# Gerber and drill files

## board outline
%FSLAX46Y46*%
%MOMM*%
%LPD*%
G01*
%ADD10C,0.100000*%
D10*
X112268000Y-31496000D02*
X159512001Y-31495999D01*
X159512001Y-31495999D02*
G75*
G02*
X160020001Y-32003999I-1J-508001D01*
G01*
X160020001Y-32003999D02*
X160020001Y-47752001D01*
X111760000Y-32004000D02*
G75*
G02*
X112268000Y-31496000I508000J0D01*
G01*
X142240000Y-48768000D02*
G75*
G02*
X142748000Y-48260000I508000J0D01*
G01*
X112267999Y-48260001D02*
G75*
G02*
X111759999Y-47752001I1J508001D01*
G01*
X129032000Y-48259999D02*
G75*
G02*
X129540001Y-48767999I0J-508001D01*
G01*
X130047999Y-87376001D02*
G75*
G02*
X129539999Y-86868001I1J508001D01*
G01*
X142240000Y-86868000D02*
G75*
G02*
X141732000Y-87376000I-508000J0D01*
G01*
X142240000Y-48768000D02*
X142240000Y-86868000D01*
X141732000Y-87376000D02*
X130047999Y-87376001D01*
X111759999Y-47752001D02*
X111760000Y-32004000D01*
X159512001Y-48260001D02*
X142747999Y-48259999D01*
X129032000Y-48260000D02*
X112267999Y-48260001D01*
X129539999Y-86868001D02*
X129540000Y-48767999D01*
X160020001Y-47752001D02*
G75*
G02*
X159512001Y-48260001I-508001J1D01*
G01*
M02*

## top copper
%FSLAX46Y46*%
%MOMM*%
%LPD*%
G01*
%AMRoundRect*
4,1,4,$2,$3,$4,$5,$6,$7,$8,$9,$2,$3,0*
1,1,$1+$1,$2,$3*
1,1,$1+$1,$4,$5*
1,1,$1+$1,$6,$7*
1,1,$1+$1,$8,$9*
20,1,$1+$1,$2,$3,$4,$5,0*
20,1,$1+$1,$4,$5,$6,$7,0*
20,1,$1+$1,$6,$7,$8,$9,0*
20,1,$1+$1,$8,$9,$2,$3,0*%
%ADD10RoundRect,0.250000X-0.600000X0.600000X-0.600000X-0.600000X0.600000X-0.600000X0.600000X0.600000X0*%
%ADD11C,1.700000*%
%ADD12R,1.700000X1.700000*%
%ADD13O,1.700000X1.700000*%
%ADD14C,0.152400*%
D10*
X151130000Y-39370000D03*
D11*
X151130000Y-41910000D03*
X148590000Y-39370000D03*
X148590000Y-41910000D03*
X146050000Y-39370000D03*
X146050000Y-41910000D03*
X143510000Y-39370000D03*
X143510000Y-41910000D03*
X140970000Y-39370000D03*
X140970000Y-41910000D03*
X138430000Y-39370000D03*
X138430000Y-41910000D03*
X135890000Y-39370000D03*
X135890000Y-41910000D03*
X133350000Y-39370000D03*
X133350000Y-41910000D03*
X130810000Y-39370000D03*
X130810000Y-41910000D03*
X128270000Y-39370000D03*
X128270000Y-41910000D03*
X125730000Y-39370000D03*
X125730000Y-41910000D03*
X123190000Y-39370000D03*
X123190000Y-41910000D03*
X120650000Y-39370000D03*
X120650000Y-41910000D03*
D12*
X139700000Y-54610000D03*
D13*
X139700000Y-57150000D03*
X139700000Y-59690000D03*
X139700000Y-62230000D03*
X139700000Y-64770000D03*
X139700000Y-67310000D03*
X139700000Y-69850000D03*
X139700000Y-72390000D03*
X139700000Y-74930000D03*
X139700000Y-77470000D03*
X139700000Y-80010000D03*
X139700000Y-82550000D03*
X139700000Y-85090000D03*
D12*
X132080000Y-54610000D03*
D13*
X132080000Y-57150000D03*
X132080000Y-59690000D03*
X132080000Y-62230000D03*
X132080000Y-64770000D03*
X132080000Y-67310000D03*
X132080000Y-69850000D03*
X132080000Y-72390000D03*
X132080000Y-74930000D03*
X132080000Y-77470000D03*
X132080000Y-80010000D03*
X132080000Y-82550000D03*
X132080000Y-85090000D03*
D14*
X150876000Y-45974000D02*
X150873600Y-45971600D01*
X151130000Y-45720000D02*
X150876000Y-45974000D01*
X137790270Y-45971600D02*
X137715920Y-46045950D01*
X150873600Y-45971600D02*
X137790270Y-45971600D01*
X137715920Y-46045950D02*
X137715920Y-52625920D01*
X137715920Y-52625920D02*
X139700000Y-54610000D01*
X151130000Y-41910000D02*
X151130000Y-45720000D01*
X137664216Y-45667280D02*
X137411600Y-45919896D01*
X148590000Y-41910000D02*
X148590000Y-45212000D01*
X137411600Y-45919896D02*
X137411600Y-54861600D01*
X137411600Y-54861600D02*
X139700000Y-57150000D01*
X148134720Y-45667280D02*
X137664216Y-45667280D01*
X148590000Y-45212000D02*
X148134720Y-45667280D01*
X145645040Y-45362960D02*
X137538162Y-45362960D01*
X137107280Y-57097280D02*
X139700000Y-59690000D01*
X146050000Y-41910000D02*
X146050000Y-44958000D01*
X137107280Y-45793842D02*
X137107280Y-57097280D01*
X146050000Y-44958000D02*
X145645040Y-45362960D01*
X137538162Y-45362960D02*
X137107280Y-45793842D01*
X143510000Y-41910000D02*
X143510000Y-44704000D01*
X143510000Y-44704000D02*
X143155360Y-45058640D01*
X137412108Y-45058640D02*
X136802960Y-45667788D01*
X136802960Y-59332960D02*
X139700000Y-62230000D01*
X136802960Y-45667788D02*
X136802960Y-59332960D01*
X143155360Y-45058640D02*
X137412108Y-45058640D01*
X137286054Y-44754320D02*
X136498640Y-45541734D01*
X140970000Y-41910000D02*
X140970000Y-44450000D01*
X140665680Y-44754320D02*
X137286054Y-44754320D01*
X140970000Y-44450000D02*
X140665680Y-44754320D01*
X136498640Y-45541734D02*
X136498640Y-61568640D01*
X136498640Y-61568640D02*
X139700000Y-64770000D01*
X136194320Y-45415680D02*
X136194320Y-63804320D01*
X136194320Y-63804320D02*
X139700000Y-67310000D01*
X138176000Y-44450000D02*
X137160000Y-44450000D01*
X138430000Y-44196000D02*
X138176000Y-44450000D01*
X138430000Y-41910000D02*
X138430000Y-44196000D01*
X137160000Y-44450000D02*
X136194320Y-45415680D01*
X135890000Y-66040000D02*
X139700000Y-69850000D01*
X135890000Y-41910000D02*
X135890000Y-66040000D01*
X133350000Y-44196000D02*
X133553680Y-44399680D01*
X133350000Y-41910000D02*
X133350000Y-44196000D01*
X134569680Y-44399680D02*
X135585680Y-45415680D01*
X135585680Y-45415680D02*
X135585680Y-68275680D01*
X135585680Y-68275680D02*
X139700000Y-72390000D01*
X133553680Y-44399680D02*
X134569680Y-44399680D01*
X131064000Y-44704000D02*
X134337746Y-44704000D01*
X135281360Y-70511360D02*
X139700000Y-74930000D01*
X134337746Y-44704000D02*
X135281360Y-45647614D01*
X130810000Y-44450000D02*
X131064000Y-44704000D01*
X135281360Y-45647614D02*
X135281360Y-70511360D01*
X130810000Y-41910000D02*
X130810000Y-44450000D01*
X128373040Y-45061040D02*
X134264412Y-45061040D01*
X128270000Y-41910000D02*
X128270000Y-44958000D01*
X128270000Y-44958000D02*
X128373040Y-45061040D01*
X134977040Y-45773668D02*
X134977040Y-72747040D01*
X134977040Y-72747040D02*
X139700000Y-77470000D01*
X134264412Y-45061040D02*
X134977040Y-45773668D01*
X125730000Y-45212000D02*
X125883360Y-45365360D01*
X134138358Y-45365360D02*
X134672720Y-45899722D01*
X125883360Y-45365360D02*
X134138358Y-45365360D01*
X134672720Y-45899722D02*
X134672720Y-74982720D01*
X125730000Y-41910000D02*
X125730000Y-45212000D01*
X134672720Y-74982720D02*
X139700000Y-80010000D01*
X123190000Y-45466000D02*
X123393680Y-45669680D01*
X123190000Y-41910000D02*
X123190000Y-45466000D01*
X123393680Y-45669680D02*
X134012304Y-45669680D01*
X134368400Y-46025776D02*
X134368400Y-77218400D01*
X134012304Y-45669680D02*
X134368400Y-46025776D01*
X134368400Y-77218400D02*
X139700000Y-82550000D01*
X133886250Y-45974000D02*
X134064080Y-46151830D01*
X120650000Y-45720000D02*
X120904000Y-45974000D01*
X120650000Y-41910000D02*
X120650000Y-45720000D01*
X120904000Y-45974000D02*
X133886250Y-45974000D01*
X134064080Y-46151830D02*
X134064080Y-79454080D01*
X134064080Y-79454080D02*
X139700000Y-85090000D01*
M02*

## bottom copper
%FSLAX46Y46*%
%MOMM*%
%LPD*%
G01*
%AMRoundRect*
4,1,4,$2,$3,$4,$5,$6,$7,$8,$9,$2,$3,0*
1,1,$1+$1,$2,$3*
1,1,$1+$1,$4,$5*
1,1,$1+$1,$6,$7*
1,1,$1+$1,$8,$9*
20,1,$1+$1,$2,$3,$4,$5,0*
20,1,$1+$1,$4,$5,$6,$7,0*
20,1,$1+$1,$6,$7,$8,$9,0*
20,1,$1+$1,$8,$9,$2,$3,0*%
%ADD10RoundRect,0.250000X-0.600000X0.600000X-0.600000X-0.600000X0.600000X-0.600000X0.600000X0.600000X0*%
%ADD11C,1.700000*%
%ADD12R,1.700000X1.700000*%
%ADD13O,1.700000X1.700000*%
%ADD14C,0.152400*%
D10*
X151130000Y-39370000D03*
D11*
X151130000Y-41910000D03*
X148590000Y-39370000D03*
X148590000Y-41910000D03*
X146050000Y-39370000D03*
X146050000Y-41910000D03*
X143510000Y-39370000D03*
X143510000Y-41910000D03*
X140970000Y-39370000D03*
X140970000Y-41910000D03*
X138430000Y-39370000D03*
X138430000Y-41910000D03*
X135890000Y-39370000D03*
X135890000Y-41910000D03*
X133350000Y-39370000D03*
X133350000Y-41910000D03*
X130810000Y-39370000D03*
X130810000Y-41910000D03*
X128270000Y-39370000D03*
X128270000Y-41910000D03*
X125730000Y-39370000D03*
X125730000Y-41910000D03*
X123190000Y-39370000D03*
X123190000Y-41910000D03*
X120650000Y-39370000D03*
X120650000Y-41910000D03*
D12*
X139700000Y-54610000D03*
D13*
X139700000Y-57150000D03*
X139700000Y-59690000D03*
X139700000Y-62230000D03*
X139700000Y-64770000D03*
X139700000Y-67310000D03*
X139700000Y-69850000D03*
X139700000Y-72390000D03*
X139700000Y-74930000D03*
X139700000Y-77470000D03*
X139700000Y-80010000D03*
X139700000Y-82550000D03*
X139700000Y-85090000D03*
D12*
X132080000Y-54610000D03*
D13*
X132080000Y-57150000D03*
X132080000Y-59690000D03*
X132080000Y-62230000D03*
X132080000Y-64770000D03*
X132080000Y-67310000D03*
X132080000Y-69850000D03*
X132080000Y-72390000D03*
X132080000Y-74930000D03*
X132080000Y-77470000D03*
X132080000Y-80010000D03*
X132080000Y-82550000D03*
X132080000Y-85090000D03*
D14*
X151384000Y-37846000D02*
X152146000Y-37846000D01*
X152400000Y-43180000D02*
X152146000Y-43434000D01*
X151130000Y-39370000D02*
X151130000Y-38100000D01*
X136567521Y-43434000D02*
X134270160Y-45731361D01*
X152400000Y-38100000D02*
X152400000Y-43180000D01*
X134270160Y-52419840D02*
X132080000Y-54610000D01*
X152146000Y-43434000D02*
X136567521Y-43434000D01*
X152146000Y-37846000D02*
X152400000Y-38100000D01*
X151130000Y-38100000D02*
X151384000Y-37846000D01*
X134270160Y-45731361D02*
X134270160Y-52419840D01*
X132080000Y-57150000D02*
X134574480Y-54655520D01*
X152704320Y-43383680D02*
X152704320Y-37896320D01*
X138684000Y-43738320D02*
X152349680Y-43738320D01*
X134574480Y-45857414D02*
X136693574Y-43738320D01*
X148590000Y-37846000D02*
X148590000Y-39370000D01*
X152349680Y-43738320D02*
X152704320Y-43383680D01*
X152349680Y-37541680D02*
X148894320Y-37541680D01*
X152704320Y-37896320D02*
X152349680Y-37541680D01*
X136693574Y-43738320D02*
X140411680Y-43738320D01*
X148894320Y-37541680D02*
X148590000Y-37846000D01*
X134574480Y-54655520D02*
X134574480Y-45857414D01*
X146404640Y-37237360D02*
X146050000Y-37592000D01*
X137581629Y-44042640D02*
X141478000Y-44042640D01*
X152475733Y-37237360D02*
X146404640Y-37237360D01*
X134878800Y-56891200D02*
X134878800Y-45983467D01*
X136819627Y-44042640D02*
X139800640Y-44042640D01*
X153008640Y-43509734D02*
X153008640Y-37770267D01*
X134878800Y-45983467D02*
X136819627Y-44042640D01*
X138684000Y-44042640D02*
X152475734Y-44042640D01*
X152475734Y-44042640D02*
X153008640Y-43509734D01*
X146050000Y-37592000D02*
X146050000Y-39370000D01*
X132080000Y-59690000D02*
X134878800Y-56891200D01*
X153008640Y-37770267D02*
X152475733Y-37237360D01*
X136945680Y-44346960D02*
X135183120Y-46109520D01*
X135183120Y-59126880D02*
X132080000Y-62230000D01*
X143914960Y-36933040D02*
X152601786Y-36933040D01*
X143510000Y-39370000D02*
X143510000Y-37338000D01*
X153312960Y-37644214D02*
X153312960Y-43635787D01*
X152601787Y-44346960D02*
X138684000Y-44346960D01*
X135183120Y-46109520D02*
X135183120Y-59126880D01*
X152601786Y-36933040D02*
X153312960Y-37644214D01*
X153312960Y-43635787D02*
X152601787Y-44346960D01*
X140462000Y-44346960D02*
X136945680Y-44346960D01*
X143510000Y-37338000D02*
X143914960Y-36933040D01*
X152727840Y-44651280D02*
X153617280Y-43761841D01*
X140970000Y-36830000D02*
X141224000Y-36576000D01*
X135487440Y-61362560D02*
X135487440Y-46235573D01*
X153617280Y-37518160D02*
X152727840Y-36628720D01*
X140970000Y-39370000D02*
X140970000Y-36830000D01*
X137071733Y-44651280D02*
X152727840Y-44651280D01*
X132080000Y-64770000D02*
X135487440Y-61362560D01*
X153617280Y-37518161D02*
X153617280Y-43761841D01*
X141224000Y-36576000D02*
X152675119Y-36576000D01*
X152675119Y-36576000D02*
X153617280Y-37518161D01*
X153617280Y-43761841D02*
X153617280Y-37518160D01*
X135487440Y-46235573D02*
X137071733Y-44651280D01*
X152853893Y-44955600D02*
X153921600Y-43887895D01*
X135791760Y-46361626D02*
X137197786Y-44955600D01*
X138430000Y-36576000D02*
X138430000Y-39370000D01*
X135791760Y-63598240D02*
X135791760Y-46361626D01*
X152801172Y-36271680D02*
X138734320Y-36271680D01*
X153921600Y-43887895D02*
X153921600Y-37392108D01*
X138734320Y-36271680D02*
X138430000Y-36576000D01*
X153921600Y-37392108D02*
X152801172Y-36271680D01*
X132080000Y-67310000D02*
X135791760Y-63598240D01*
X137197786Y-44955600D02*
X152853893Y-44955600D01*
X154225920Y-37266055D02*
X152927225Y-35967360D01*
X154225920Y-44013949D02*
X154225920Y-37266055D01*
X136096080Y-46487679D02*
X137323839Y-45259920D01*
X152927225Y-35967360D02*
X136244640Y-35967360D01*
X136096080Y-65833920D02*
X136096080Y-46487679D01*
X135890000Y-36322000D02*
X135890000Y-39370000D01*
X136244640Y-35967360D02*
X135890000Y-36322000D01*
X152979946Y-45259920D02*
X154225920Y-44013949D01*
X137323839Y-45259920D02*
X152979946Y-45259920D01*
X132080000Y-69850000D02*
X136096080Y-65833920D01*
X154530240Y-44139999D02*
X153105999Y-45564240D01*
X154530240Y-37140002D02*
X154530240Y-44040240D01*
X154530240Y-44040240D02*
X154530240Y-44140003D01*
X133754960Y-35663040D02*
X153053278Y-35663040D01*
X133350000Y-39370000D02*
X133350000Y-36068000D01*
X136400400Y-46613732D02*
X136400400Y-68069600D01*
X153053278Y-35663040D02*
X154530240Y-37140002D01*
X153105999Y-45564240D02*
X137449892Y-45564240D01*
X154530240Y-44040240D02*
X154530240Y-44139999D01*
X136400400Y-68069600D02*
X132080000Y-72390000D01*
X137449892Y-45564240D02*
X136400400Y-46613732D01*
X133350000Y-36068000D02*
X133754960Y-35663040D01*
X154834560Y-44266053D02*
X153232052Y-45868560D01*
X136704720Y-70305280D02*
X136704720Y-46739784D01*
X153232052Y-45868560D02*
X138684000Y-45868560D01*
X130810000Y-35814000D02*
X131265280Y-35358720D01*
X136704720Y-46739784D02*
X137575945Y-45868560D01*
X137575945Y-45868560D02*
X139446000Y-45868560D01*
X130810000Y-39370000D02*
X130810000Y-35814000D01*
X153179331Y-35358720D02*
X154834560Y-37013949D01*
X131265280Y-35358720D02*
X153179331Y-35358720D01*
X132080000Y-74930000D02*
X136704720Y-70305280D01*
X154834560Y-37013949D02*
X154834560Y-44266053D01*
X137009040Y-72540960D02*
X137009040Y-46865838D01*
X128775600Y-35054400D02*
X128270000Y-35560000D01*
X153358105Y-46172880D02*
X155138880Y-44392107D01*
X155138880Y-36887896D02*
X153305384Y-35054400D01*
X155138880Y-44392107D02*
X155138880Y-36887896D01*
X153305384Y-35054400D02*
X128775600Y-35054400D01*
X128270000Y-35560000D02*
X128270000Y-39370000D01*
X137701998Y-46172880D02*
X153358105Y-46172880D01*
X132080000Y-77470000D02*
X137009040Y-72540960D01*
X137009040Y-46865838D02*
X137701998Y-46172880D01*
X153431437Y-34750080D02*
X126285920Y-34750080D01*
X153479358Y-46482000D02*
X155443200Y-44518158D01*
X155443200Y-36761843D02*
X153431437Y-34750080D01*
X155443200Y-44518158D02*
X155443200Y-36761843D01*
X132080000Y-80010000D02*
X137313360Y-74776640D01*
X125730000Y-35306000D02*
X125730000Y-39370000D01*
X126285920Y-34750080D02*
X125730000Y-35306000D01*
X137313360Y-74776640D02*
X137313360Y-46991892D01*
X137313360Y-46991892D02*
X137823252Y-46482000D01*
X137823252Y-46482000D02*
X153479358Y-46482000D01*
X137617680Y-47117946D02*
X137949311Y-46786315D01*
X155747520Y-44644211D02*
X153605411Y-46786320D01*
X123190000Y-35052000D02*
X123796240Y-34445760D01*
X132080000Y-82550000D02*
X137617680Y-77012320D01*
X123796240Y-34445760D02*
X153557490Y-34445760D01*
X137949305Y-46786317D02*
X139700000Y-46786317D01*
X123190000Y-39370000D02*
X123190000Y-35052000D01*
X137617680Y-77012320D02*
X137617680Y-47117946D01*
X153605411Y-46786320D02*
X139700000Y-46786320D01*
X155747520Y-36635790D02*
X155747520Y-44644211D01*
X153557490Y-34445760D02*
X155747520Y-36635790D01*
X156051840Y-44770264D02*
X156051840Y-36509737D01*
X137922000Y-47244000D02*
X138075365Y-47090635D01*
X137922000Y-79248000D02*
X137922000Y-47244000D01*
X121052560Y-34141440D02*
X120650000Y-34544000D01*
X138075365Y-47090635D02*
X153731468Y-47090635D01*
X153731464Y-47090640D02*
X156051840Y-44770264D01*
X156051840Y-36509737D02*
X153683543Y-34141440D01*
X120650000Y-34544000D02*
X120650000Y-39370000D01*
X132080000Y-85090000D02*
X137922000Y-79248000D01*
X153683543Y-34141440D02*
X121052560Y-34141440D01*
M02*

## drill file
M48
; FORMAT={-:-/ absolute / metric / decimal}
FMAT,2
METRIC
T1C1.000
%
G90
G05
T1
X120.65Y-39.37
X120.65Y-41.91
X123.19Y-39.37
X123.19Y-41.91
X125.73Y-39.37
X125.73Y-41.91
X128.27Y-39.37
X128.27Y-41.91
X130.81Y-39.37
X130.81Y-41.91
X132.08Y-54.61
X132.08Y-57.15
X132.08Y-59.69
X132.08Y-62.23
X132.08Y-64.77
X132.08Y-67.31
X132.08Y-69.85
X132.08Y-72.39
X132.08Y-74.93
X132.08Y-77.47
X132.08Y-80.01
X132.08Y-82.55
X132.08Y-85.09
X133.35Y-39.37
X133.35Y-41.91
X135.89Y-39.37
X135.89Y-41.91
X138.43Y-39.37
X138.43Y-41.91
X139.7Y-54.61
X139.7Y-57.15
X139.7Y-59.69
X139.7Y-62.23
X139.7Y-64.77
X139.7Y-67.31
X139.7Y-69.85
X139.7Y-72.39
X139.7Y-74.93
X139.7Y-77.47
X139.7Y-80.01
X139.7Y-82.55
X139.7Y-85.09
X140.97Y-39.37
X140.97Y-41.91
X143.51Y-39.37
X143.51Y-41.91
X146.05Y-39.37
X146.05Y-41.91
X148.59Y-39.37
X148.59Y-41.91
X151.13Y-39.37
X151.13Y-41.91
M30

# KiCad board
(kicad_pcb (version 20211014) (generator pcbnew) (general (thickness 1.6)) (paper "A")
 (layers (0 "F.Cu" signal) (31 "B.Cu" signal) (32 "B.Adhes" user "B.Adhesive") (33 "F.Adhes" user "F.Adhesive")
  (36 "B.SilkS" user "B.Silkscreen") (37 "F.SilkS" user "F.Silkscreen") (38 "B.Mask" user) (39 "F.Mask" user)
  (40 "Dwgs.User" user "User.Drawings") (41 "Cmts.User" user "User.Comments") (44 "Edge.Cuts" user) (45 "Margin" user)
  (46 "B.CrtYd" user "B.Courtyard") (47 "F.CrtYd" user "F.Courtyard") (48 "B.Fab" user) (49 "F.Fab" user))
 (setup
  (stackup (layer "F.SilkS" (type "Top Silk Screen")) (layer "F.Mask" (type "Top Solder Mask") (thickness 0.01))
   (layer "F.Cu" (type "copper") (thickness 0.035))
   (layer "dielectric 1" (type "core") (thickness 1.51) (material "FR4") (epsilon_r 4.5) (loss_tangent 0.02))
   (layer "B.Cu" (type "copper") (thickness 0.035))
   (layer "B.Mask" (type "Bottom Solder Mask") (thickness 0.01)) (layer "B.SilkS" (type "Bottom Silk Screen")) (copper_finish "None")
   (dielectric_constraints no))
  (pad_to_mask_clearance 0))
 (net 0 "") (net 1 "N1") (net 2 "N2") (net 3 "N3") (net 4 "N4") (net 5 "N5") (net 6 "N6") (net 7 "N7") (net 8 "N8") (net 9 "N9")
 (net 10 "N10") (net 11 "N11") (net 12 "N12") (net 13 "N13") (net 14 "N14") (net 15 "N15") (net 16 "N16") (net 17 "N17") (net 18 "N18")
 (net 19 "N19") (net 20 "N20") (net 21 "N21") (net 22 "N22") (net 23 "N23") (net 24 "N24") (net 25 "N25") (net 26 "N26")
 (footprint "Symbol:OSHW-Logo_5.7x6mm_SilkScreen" (layer "F.Cu") (at 135.89 49.53)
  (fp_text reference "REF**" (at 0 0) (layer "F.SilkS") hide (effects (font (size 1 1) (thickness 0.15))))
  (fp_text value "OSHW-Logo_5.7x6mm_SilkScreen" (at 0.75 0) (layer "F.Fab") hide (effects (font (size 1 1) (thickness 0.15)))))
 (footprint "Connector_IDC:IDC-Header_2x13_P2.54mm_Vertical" (layer "F.Cu") (at 151.13 39.37 -90)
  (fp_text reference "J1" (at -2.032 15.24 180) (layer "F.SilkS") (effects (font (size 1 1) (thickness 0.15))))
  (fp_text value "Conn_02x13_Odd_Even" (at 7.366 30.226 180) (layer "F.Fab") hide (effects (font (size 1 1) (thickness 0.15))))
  (pad "1" thru_hole roundrect locked (at 0 0 270) (size 1.7 1.7) (drill 1) (layers *.Cu *.Mask) (roundrect_rratio 0.1470588235)
   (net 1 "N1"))
  (pad "2" thru_hole circle locked (at 2.54 0 270) (size 1.7 1.7) (drill 1) (layers *.Cu *.Mask) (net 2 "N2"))
  (pad "3" thru_hole circle locked (at 0 2.54 270) (size 1.7 1.7) (drill 1) (layers *.Cu *.Mask) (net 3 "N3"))
  (pad "4" thru_hole circle locked (at 2.54 2.54 270) (size 1.7 1.7) (drill 1) (layers *.Cu *.Mask) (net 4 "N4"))
  (pad "5" thru_hole circle locked (at 0 5.08 270) (size 1.7 1.7) (drill 1) (layers *.Cu *.Mask) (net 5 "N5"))
  (pad "6" thru_hole circle locked (at 2.54 5.08 270) (size 1.7 1.7) (drill 1) (layers *.Cu *.Mask) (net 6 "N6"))
  (pad "7" thru_hole circle locked (at 0 7.62 270) (size 1.7 1.7) (drill 1) (layers *.Cu *.Mask) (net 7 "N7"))
  (pad "8" thru_hole circle locked (at 2.54 7.62 270) (size 1.7 1.7) (drill 1) (layers *.Cu *.Mask) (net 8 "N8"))
  (pad "9" thru_hole circle locked (at 0 10.16 270) (size 1.7 1.7) (drill 1) (layers *.Cu *.Mask) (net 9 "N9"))
  (pad "10" thru_hole circle locked (at 2.54 10.16 270) (size 1.7 1.7) (drill 1) (layers *.Cu *.Mask) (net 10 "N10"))
  (pad "11" thru_hole circle locked (at 0 12.7 270) (size 1.7 1.7) (drill 1) (layers *.Cu *.Mask) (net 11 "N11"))
  (pad "12" thru_hole circle locked (at 2.54 12.7 270) (size 1.7 1.7) (drill 1) (layers *.Cu *.Mask) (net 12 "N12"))
  (pad "13" thru_hole circle locked (at 0 15.24 270) (size 1.7 1.7) (drill 1) (layers *.Cu *.Mask) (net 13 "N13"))
  (pad "14" thru_hole circle locked (at 2.54 15.24 270) (size 1.7 1.7) (drill 1) (layers *.Cu *.Mask) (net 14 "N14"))
  (pad "15" thru_hole circle locked (at 0 17.78 270) (size 1.7 1.7) (drill 1) (layers *.Cu *.Mask) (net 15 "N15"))
  (pad "16" thru_hole circle locked (at 2.54 17.78 270) (size 1.7 1.7) (drill 1) (layers *.Cu *.Mask) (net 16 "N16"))
  (pad "17" thru_hole circle locked (at 0 20.32 270) (size 1.7 1.7) (drill 1) (layers *.Cu *.Mask) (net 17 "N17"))
  (pad "18" thru_hole circle locked (at 2.54 20.32 270) (size 1.7 1.7) (drill 1) (layers *.Cu *.Mask) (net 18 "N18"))
  (pad "19" thru_hole circle locked (at 0 22.86 270) (size 1.7 1.7) (drill 1) (layers *.Cu *.Mask) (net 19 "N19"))
  (pad "20" thru_hole circle locked (at 2.54 22.86 270) (size 1.7 1.7) (drill 1) (layers *.Cu *.Mask) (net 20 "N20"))
  (pad "21" thru_hole circle locked (at 0 25.4 270) (size 1.7 1.7) (drill 1) (layers *.Cu *.Mask) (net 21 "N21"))
  (pad "22" thru_hole circle locked (at 2.54 25.4 270) (size 1.7 1.7) (drill 1) (layers *.Cu *.Mask) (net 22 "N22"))
  (pad "23" thru_hole circle locked (at 0 27.94 270) (size 1.7 1.7) (drill 1) (layers *.Cu *.Mask) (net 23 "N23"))
  (pad "24" thru_hole circle locked (at 2.54 27.94 270) (size 1.7 1.7) (drill 1) (layers *.Cu *.Mask) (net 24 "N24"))
  (pad "25" thru_hole circle locked (at 0 30.48 270) (size 1.7 1.7) (drill 1) (layers *.Cu *.Mask) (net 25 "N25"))
  (pad "26" thru_hole circle locked (at 2.54 30.48 270) (size 1.7 1.7) (drill 1) (layers *.Cu *.Mask) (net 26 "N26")))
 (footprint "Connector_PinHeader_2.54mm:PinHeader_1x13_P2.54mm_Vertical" (layer "B.Cu") (at 139.7 54.61 180)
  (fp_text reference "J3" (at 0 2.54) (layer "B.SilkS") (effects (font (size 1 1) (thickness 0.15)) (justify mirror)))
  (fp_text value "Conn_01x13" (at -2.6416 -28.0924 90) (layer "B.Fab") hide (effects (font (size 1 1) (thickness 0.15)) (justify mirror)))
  (pad "1" thru_hole rect locked (at 0 0 180) (size 1.7 1.7) (drill 1) (layers *.Cu *.Mask) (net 2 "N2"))
  (pad "2" thru_hole oval locked (at 0 -2.54 180) (size 1.7 1.7) (drill 1) (layers *.Cu *.Mask) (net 4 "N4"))
  (pad "3" thru_hole oval locked (at 0 -5.08 180) (size 1.7 1.7) (drill 1) (layers *.Cu *.Mask) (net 6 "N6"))
  (pad "4" thru_hole oval locked (at 0 -7.62 180) (size 1.7 1.7) (drill 1) (layers *.Cu *.Mask) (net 8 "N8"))
  (pad "5" thru_hole oval locked (at 0 -10.16 180) (size 1.7 1.7) (drill 1) (layers *.Cu *.Mask) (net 10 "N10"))
  (pad "6" thru_hole oval locked (at 0 -12.7 180) (size 1.7 1.7) (drill 1) (layers *.Cu *.Mask) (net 12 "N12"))
  (pad "7" thru_hole oval locked (at 0 -15.24 180) (size 1.7 1.7) (drill 1) (layers *.Cu *.Mask) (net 14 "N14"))
  (pad "8" thru_hole oval locked (at 0 -17.78 180) (size 1.7 1.7) (drill 1) (layers *.Cu *.Mask) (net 16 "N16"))
  (pad "9" thru_hole oval locked (at 0 -20.32 180) (size 1.7 1.7) (drill 1) (layers *.Cu *.Mask) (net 18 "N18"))
  (pad "10" thru_hole oval locked (at 0 -22.86 180) (size 1.7 1.7) (drill 1) (layers *.Cu *.Mask) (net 20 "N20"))
  (pad "11" thru_hole oval locked (at 0 -25.4 180) (size 1.7 1.7) (drill 1) (layers *.Cu *.Mask) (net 22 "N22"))
  (pad "12" thru_hole oval locked (at 0 -27.94 180) (size 1.7 1.7) (drill 1) (layers *.Cu *.Mask) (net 24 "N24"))
  (pad "13" thru_hole oval locked (at 0 -30.48 180) (size 1.7 1.7) (drill 1) (layers *.Cu *.Mask) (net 26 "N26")))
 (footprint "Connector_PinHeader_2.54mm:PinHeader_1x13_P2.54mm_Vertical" (layer "B.Cu") (at 132.08 54.61 180)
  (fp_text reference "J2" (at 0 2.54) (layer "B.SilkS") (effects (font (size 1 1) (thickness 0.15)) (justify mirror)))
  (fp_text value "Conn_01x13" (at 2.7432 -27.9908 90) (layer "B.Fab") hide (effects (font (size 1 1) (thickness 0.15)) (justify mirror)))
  (pad "1" thru_hole rect locked (at 0 0 180) (size 1.7 1.7) (drill 1) (layers *.Cu *.Mask) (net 1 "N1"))
  (pad "2" thru_hole oval locked (at 0 -2.54 180) (size 1.7 1.7) (drill 1) (layers *.Cu *.Mask) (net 3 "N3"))
  (pad "3" thru_hole oval locked (at 0 -5.08 180) (size 1.7 1.7) (drill 1) (layers *.Cu *.Mask) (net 5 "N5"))
  (pad "4" thru_hole oval locked (at 0 -7.62 180) (size 1.7 1.7) (drill 1) (layers *.Cu *.Mask) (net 7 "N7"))
  (pad "5" thru_hole oval locked (at 0 -10.16 180) (size 1.7 1.7) (drill 1) (layers *.Cu *.Mask) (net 9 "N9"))
  (pad "6" thru_hole oval locked (at 0 -12.7 180) (size 1.7 1.7) (drill 1) (layers *.Cu *.Mask) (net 11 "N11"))
  (pad "7" thru_hole oval locked (at 0 -15.24 180) (size 1.7 1.7) (drill 1) (layers *.Cu *.Mask) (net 13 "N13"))
  (pad "8" thru_hole oval locked (at 0 -17.78 180) (size 1.7 1.7) (drill 1) (layers *.Cu *.Mask) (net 15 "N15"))
  (pad "9" thru_hole oval locked (at 0 -20.32 180) (size 1.7 1.7) (drill 1) (layers *.Cu *.Mask) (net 17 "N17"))
  (pad "10" thru_hole oval locked (at 0 -22.86 180) (size 1.7 1.7) (drill 1) (layers *.Cu *.Mask) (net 19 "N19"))
  (pad "11" thru_hole oval locked (at 0 -25.4 180) (size 1.7 1.7) (drill 1) (layers *.Cu *.Mask) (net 21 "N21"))
  (pad "12" thru_hole oval locked (at 0 -27.94 180) (size 1.7 1.7) (drill 1) (layers *.Cu *.Mask) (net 23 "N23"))
  (pad "13" thru_hole oval locked (at 0 -30.48 180) (size 1.7 1.7) (drill 1) (layers *.Cu *.Mask) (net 25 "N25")))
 (gr_line (start 112.268 31.496) (end 159.512001 31.495999) (layer "Edge.Cuts") (width 0.1))
 (gr_arc (start 159.512001 31.495999) (mid 159.871211 31.644789) (end 160.020001 32.003999) (layer "Edge.Cuts") (width 0.1))
 (gr_line (start 160.020001 32.003999) (end 160.020001 47.752001) (layer "Edge.Cuts") (width 0.1))
 (gr_arc (start 111.76 32.004) (mid 111.90879 31.64479) (end 112.268 31.496) (layer "Edge.Cuts") (width 0.1))
 (gr_arc (start 142.24 48.768) (mid 142.38879 48.40879) (end 142.748 48.26) (layer "Edge.Cuts") (width 0.1))
 (gr_arc (start 112.267999 48.260001) (mid 111.908789 48.111211) (end 111.759999 47.752001) (layer "Edge.Cuts") (width 0.1))
 (gr_arc (start 129.032 48.259999) (mid 129.39121 48.408789) (end 129.54 48.767999) (layer "Edge.Cuts") (width 0.1))
 (gr_arc (start 130.047999 87.376001) (mid 129.688789 87.227211) (end 129.539999 86.868001) (layer "Edge.Cuts") (width 0.1))
 (gr_arc (start 142.24 86.868) (mid 142.09121 87.22721) (end 141.732 87.376) (layer "Edge.Cuts") (width 0.1))
 (gr_line (start 142.24 48.768) (end 142.24 86.868) (layer "Edge.Cuts") (width 0.1))
 (gr_line (start 141.732 87.376) (end 130.047999 87.376001) (layer "Edge.Cuts") (width 0.1))
 (gr_line (start 111.759999 47.752001) (end 111.76 32.004) (layer "Edge.Cuts") (width 0.1))
 (gr_line (start 159.512001 48.260001) (end 142.747999 48.259999) (layer "Edge.Cuts") (width 0.1))
 (gr_line (start 129.032 48.26) (end 112.267999 48.260001) (layer "Edge.Cuts") (width 0.1))
 (gr_line (start 129.539999 86.868001) (end 129.54 48.767999) (layer "Edge.Cuts") (width 0.1))
 (gr_arc (start 160.020001 47.752001) (mid 159.871211 48.111211) (end 159.512001 48.260001) (layer "Edge.Cuts") (width 0.1))
 (segment (start 151.384 37.846) (end 152.146 37.846) (width 0.1524) (layer "B.Cu") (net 1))
 (segment (start 152.4 43.18) (end 152.146 43.434) (width 0.1524) (layer "B.Cu") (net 1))
 (segment (start 151.13 39.37) (end 151.13 38.1) (width 0.1524) (layer "B.Cu") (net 1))
 (segment (start 136.567521 43.434) (end 134.27016 45.731361) (width 0.1524) (layer "B.Cu") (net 1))
 (segment (start 152.4 38.1) (end 152.4 43.18) (width 0.1524) (layer "B.Cu") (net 1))
 (segment (start 134.27016 52.41984) (end 132.08 54.61) (width 0.1524) (layer "B.Cu") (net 1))
 (segment (start 152.146 43.434) (end 136.567521 43.434) (width 0.1524) (layer "B.Cu") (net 1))
 (segment (start 152.146 37.846) (end 152.4 38.1) (width 0.1524) (layer "B.Cu") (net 1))
 (segment (start 151.13 38.1) (end 151.384 37.846) (width 0.1524) (layer "B.Cu") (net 1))
 (segment (start 134.27016 45.731361) (end 134.27016 52.41984) (width 0.1524) (layer "B.Cu") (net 1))
 (segment (start 132.08 57.15) (end 134.57448 54.65552) (width 0.1524) (layer "B.Cu") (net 3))
 (segment (start 152.70432 43.38368) (end 152.70432 37.89632) (width 0.1524) (layer "B.Cu") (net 3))
 (segment (start 138.684 43.73832) (end 152.34968 43.73832) (width 0.1524) (layer "B.Cu") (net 3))
 (segment (start 134.57448 45.857414) (end 136.693574 43.73832) (width 0.1524) (layer "B.Cu") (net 3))
 (segment (start 148.59 37.846) (end 148.59 39.37) (width 0.1524) (layer "B.Cu") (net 3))
 (segment (start 152.34968 43.73832) (end 152.70432 43.38368) (width 0.1524) (layer "B.Cu") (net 3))
 (segment (start 152.34968 37.54168) (end 148.89432 37.54168) (width 0.1524) (layer "B.Cu") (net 3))
 (segment (start 152.70432 37.89632) (end 152.34968 37.54168) (width 0.1524) (layer "B.Cu") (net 3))
 (segment (start 136.693574 43.73832) (end 140.41168 43.73832) (width 0.1524) (layer "B.Cu") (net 3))
 (segment (start 148.89432 37.54168) (end 148.59 37.846) (width 0.1524) (layer "B.Cu") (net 3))
 (segment (start 134.57448 54.65552) (end 134.57448 45.857414) (width 0.1524) (layer "B.Cu") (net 3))
 (segment (start 146.40464 37.23736) (end 146.05 37.592) (width 0.1524) (layer "B.Cu") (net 5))
 (segment (start 137.581629 44.04264) (end 141.478 44.04264) (width 0.1524) (layer "B.Cu") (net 5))
 (segment (start 152.475733 37.23736) (end 146.40464 37.23736) (width 0.1524) (layer "B.Cu") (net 5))
 (segment (start 134.8788 56.8912) (end 134.8788 45.983467) (width 0.1524) (layer "B.Cu") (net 5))
 (segment (start 136.819627 44.04264) (end 139.80064 44.04264) (width 0.1524) (layer "B.Cu") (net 5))
 (segment (start 153.00864 43.509734) (end 153.00864 37.770267) (width 0.1524) (layer "B.Cu") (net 5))
 (segment (start 134.8788 45.983467) (end 136.819627 44.04264) (width 0.1524) (layer "B.Cu") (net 5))
 (segment (start 138.684 44.04264) (end 152.475734 44.04264) (width 0.1524) (layer "B.Cu") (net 5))
 (segment (start 152.475734 44.04264) (end 153.00864 43.509734) (width 0.1524) (layer "B.Cu") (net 5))
 (segment (start 146.05 37.592) (end 146.05 39.37) (width 0.1524) (layer "B.Cu") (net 5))
 (segment (start 132.08 59.69) (end 134.8788 56.8912) (width 0.1524) (layer "B.Cu") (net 5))
 (segment (start 153.00864 37.770267) (end 152.475733 37.23736) (width 0.1524) (layer "B.Cu") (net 5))
 (segment (start 136.94568 44.34696) (end 135.18312 46.10952) (width 0.1524) (layer "B.Cu") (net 7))
 (segment (start 135.18312 59.12688) (end 132.08 62.23) (width 0.1524) (layer "B.Cu") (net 7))
 (segment (start 143.91496 36.93304) (end 152.601786 36.93304) (width 0.1524) (layer "B.Cu") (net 7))
 (segment (start 143.51 39.37) (end 143.51 37.338) (width 0.1524) (layer "B.Cu") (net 7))
 (segment (start 153.31296 37.644214) (end 153.31296 43.635787) (width 0.1524) (layer "B.Cu") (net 7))
 (segment (start 152.601787 44.34696) (end 138.684 44.34696) (width 0.1524) (layer "B.Cu") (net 7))
 (segment (start 135.18312 46.10952) (end 135.18312 59.12688) (width 0.1524) (layer "B.Cu") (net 7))
 (segment (start 152.601786 36.93304) (end 153.31296 37.644214) (width 0.1524) (layer "B.Cu") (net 7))
 (segment (start 153.31296 43.635787) (end 152.601787 44.34696) (width 0.1524) (layer "B.Cu") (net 7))
 (segment (start 140.462 44.34696) (end 136.94568 44.34696) (width 0.1524) (layer "B.Cu") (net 7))
 (segment (start 143.51 37.338) (end 143.91496 36.93304) (width 0.1524) (layer "B.Cu") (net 7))
 (segment (start 152.72784 44.65128) (end 153.61728 43.761841) (width 0.1524) (layer "B.Cu") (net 9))
 (segment (start 140.97 36.83) (end 141.224 36.576) (width 0.1524) (layer "B.Cu") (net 9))
 (segment (start 135.48744 61.36256) (end 135.48744 46.235573) (width 0.1524) (layer "B.Cu") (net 9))
 (segment (start 153.61728 37.51816) (end 152.72784 36.62872) (width 0.1524) (layer "B.Cu") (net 9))
 (segment (start 140.97 39.37) (end 140.97 36.83) (width 0.1524) (layer "B.Cu") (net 9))
 (segment (start 137.071733 44.65128) (end 152.72784 44.65128) (width 0.1524) (layer "B.Cu") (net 9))
 (segment (start 132.08 64.77) (end 135.48744 61.36256) (width 0.1524) (layer "B.Cu") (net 9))
 (segment (start 153.61728 37.518161) (end 153.61728 43.761841) (width 0.1524) (layer "B.Cu") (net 9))
 (segment (start 141.224 36.576) (end 152.675119 36.576) (width 0.1524) (layer "B.Cu") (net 9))
 (segment (start 152.675119 36.576) (end 153.61728 37.518161) (width 0.1524) (layer "B.Cu") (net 9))
 (segment (start 153.61728 43.761841) (end 153.61728 37.51816) (width 0.1524) (layer "B.Cu") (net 9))
 (segment (start 135.48744 46.235573) (end 137.071733 44.65128) (width 0.1524) (layer "B.Cu") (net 9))
 (segment (start 152.853893 44.9556) (end 153.9216 43.887895) (width 0.1524) (layer "B.Cu") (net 11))
 (segment (start 135.79176 46.361626) (end 137.197786 44.9556) (width 0.1524) (layer "B.Cu") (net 11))
 (segment (start 138.43 36.576) (end 138.43 39.37) (width 0.1524) (layer "B.Cu") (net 11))
 (segment (start 135.79176 63.59824) (end 135.79176 46.361626) (width 0.1524) (layer "B.Cu") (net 11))
 (segment (start 152.801172 36.27168) (end 138.73432 36.27168) (width 0.1524) (layer "B.Cu") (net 11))
 (segment (start 153.9216 43.887895) (end 153.9216 37.392108) (width 0.1524) (layer "B.Cu") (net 11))
 (segment (start 138.73432 36.27168) (end 138.43 36.576) (width 0.1524) (layer "B.Cu") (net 11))
 (segment (start 153.9216 37.392108) (end 152.801172 36.27168) (width 0.1524) (layer "B.Cu") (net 11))
 (segment (start 132.08 67.31) (end 135.79176 63.59824) (width 0.1524) (layer "B.Cu") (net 11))
 (segment (start 137.197786 44.9556) (end 152.853893 44.9556) (width 0.1524) (layer "B.Cu") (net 11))
 (segment (start 154.22592 37.266055) (end 152.927225 35.96736) (width 0.1524) (layer "B.Cu") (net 13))
 (segment (start 154.22592 44.013949) (end 154.22592 37.266055) (width 0.1524) (layer "B.Cu") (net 13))
 (segment (start 136.09608 46.487679) (end 137.323839 45.25992) (width 0.1524) (layer "B.Cu") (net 13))
 (segment (start 152.927225 35.96736) (end 136.24464 35.96736) (width 0.1524) (layer "B.Cu") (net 13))
 (segment (start 136.09608 65.83392) (end 136.09608 46.487679) (width 0.1524) (layer "B.Cu") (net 13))
 (segment (start 135.89 36.322) (end 135.89 39.37) (width 0.1524) (layer "B.Cu") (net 13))
 (segment (start 136.24464 35.96736) (end 135.89 36.322) (width 0.1524) (layer "B.Cu") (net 13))
 (segment (start 152.979946 45.25992) (end 154.22592 44.013949) (width 0.1524) (layer "B.Cu") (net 13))
 (segment (start 137.323839 45.25992) (end 152.979946 45.25992) (width 0.1524) (layer "B.Cu") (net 13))
 (segment (start 132.08 69.85) (end 136.09608 65.83392) (width 0.1524) (layer "B.Cu") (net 13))
 (segment (start 154.53024 44.139999) (end 153.105999 45.56424) (width 0.1524) (layer "B.Cu") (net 15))
 (segment (start 154.53024 37.140002) (end 154.53024 44.04024) (width 0.1524) (layer "B.Cu") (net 15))
 (segment (start 154.53024 44.04024) (end 154.53024 44.140003) (width 0.1524) (layer "B.Cu") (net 15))
 (segment (start 133.75496 35.66304) (end 153.053278 35.66304) (width 0.1524) (layer "B.Cu") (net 15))
 (segment (start 133.35 39.37) (end 133.35 36.068) (width 0.1524) (layer "B.Cu") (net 15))
 (segment (start 136.4004 46.613732) (end 136.4004 68.0696) (width 0.1524) (layer "B.Cu") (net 15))
 (segment (start 153.053278 35.66304) (end 154.53024 37.140002) (width 0.1524) (layer "B.Cu") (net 15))
 (segment (start 153.105999 45.56424) (end 137.449892 45.56424) (width 0.1524) (layer "B.Cu") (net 15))
 (segment (start 154.53024 44.04024) (end 154.53024 44.139999) (width 0.1524) (layer "B.Cu") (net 15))
 (segment (start 136.4004 68.0696) (end 132.08 72.39) (width 0.1524) (layer "B.Cu") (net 15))
 (segment (start 137.449892 45.56424) (end 136.4004 46.613732) (width 0.1524) (layer "B.Cu") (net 15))
 (segment (start 133.35 36.068) (end 133.75496 35.66304) (width 0.1524) (layer "B.Cu") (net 15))
 (segment (start 154.83456 44.266053) (end 153.232052 45.86856) (width 0.1524) (layer "B.Cu") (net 17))
 (segment (start 136.70472 70.30528) (end 136.70472 46.739784) (width 0.1524) (layer "B.Cu") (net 17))
 (segment (start 153.232052 45.86856) (end 138.684 45.86856) (width 0.1524) (layer "B.Cu") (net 17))
 (segment (start 130.81 35.814) (end 131.26528 35.35872) (width 0.1524) (layer "B.Cu") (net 17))
 (segment (start 136.70472 46.739784) (end 137.575945 45.86856) (width 0.1524) (layer "B.Cu") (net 17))
 (segment (start 137.575945 45.86856) (end 139.446 45.86856) (width 0.1524) (layer "B.Cu") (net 17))
 (segment (start 130.81 39.37) (end 130.81 35.814) (width 0.1524) (layer "B.Cu") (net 17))
 (segment (start 153.179331 35.35872) (end 154.83456 37.013949) (width 0.1524) (layer "B.Cu") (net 17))
 (segment (start 131.26528 35.35872) (end 153.179331 35.35872) (width 0.1524) (layer "B.Cu") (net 17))
 (segment (start 132.08 74.93) (end 136.70472 70.30528) (width 0.1524) (layer "B.Cu") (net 17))
 (segment (start 154.83456 37.013949) (end 154.83456 44.266053) (width 0.1524) (layer "B.Cu") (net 17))
 (segment (start 137.00904 72.54096) (end 137.00904 46.865838) (width 0.1524) (layer "B.Cu") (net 19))
 (segment (start 128.7756 35.0544) (end 128.27 35.56) (width 0.1524) (layer "B.Cu") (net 19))
 (segment (start 153.358105 46.17288) (end 155.13888 44.392107) (width 0.1524) (layer "B.Cu") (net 19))
 (segment (start 155.13888 36.887896) (end 153.305384 35.0544) (width 0.1524) (layer "B.Cu") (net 19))
 (segment (start 155.13888 44.392107) (end 155.13888 36.887896) (width 0.1524) (layer "B.Cu") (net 19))
 (segment (start 153.305384 35.0544) (end 128.7756 35.0544) (width 0.1524) (layer "B.Cu") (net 19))
 (segment (start 128.27 35.56) (end 128.27 39.37) (width 0.1524) (layer "B.Cu") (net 19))
 (segment (start 137.701998 46.17288) (end 153.358105 46.17288) (width 0.1524) (layer "B.Cu") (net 19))
 (segment (start 132.08 77.47) (end 137.00904 72.54096) (width 0.1524) (layer "B.Cu") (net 19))
 (segment (start 137.00904 46.865838) (end 137.701998 46.17288) (width 0.1524) (layer "B.Cu") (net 19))
 (segment (start 153.431437 34.75008) (end 126.28592 34.75008) (width 0.1524) (layer "B.Cu") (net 21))
 (segment (start 153.479358 46.482) (end 155.4432 44.518158) (width 0.1524) (layer "B.Cu") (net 21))
 (segment (start 155.4432 36.761843) (end 153.431437 34.75008) (width 0.1524) (layer "B.Cu") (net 21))
 (segment (start 155.4432 44.518158) (end 155.4432 36.761843) (width 0.1524) (layer "B.Cu") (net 21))
 (segment (start 132.08 80.01) (end 137.31336 74.77664) (width 0.1524) (layer "B.Cu") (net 21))
 (segment (start 125.73 35.306) (end 125.73 39.37) (width 0.1524) (layer "B.Cu") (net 21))
 (segment (start 126.28592 34.75008) (end 125.73 35.306) (width 0.1524) (layer "B.Cu") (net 21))
 (segment (start 137.31336 74.77664) (end 137.31336 46.991892) (width 0.1524) (layer "B.Cu") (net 21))
 (segment (start 137.31336 46.991892) (end 137.823252 46.482) (width 0.1524) (layer "B.Cu") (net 21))
 (segment (start 137.823252 46.482) (end 153.479358 46.482) (width 0.1524) (layer "B.Cu") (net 21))
 (segment (start 137.61768 47.117946) (end 137.949311 46.786315) (width 0.1524) (layer "B.Cu") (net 23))
 (segment (start 155.74752 44.644211) (end 153.605411 46.78632) (width 0.1524) (layer "B.Cu") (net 23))
 (segment (start 123.19 35.052) (end 123.79624 34.44576) (width 0.1524) (layer "B.Cu") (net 23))
 (segment (start 132.08 82.55) (end 137.61768 77.01232) (width 0.1524) (layer "B.Cu") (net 23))
 (segment (start 123.79624 34.44576) (end 153.55749 34.44576) (width 0.1524) (layer "B.Cu") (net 23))
 (segment (start 137.949305 46.786317) (end 139.7 46.786317) (width 0.1524) (layer "B.Cu") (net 23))
 (segment (start 123.19 39.37) (end 123.19 35.052) (width 0.1524) (layer "B.Cu") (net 23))
 (segment (start 137.61768 77.01232) (end 137.61768 47.117946) (width 0.1524) (layer "B.Cu") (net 23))
 (segment (start 153.605411 46.78632) (end 139.7 46.78632) (width 0.1524) (layer "B.Cu") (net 23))
 (segment (start 155.74752 36.63579) (end 155.74752 44.644211) (width 0.1524) (layer "B.Cu") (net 23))
 (segment (start 153.55749 34.44576) (end 155.74752 36.63579) (width 0.1524) (layer "B.Cu") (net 23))
 (segment (start 156.05184 44.770264) (end 156.05184 36.509737) (width 0.1524) (layer "B.Cu") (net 25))
 (segment (start 137.922 47.244) (end 138.075365 47.090635) (width 0.1524) (layer "B.Cu") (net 25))
 (segment (start 137.922 79.248) (end 137.922 47.244) (width 0.1524) (layer "B.Cu") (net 25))
 (segment (start 121.05256 34.14144) (end 120.65 34.544) (width 0.1524) (layer "B.Cu") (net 25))
 (segment (start 138.075365 47.090635) (end 153.731468 47.090635) (width 0.1524) (layer "B.Cu") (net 25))
 (segment (start 153.731464 47.09064) (end 156.05184 44.770264) (width 0.1524) (layer "B.Cu") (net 25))
 (segment (start 156.05184 36.509737) (end 153.683543 34.14144) (width 0.1524) (layer "B.Cu") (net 25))
 (segment (start 120.65 34.544) (end 120.65 39.37) (width 0.1524) (layer "B.Cu") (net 25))
 (segment (start 132.08 85.09) (end 137.922 79.248) (width 0.1524) (layer "B.Cu") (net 25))
 (segment (start 153.683543 34.14144) (end 121.05256 34.14144) (width 0.1524) (layer "B.Cu") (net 25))
 (segment (start 150.876 45.974) (end 150.8736 45.9716) (width 0.1524) (layer "F.Cu") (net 2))
 (segment (start 151.13 45.72) (end 150.876 45.974) (width 0.1524) (layer "F.Cu") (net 2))
 (segment (start 137.79027 45.9716) (end 137.71592 46.04595) (width 0.1524) (layer "F.Cu") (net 2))
 (segment (start 150.8736 45.9716) (end 137.79027 45.9716) (width 0.1524) (layer "F.Cu") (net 2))
 (segment (start 137.71592 46.04595) (end 137.71592 52.62592) (width 0.1524) (layer "F.Cu") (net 2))
 (segment (start 137.71592 52.62592) (end 139.7 54.61) (width 0.1524) (layer "F.Cu") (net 2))
 (segment (start 151.13 41.91) (end 151.13 45.72) (width 0.1524) (layer "F.Cu") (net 2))
 (segment (start 137.664216 45.66728) (end 137.4116 45.919896) (width 0.1524) (layer "F.Cu") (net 4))
 (segment (start 148.59 41.91) (end 148.59 45.212) (width 0.1524) (layer "F.Cu") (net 4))
 (segment (start 137.4116 45.919896) (end 137.4116 54.8616) (width 0.1524) (layer "F.Cu") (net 4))
 (segment (start 137.4116 54.8616) (end 139.7 57.15) (width 0.1524) (layer "F.Cu") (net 4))
 (segment (start 148.13472 45.66728) (end 137.664216 45.66728) (width 0.1524) (layer "F.Cu") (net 4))
 (segment (start 148.59 45.212) (end 148.13472 45.66728) (width 0.1524) (layer "F.Cu") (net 4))
 (segment (start 145.64504 45.36296) (end 137.538162 45.36296) (width 0.1524) (layer "F.Cu") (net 6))
 (segment (start 137.10728 57.09728) (end 139.7 59.69) (width 0.1524) (layer "F.Cu") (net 6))
 (segment (start 146.05 41.91) (end 146.05 44.958) (width 0.1524) (layer "F.Cu") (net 6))
 (segment (start 137.10728 45.793842) (end 137.10728 57.09728) (width 0.1524) (layer "F.Cu") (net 6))
 (segment (start 146.05 44.958) (end 145.64504 45.36296) (width 0.1524) (layer "F.Cu") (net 6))
 (segment (start 137.538162 45.36296) (end 137.10728 45.793842) (width 0.1524) (layer "F.Cu") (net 6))
 (segment (start 143.51 41.91) (end 143.51 44.704) (width 0.1524) (layer "F.Cu") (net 8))
 (segment (start 143.51 44.704) (end 143.15536 45.05864) (width 0.1524) (layer "F.Cu") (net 8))
 (segment (start 137.412108 45.05864) (end 136.80296 45.667788) (width 0.1524) (layer "F.Cu") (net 8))
 (segment (start 136.80296 59.33296) (end 139.7 62.23) (width 0.1524) (layer "F.Cu") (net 8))
 (segment (start 136.80296 45.667788) (end 136.80296 59.33296) (width 0.1524) (layer "F.Cu") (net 8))
 (segment (start 143.15536 45.05864) (end 137.412108 45.05864) (width 0.1524) (layer "F.Cu") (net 8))
 (segment (start 137.286054 44.75432) (end 136.49864 45.541734) (width 0.1524) (layer "F.Cu") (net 10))
 (segment (start 140.97 41.91) (end 140.97 44.45) (width 0.1524) (layer "F.Cu") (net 10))
 (segment (start 140.66568 44.75432) (end 137.286054 44.75432) (width 0.1524) (layer "F.Cu") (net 10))
 (segment (start 140.97 44.45) (end 140.66568 44.75432) (width 0.1524) (layer "F.Cu") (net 10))
 (segment (start 136.49864 45.541734) (end 136.49864 61.56864) (width 0.1524) (layer "F.Cu") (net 10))
 (segment (start 136.49864 61.56864) (end 139.7 64.77) (width 0.1524) (layer "F.Cu") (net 10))
 (segment (start 136.19432 45.41568) (end 136.19432 63.80432) (width 0.1524) (layer "F.Cu") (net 12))
 (segment (start 136.19432 63.80432) (end 139.7 67.31) (width 0.1524) (layer "F.Cu") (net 12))
 (segment (start 138.176 44.45) (end 137.16 44.45) (width 0.1524) (layer "F.Cu") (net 12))
 (segment (start 138.43 44.196) (end 138.176 44.45) (width 0.1524) (layer "F.Cu") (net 12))
 (segment (start 138.43 41.91) (end 138.43 44.196) (width 0.1524) (layer "F.Cu") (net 12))
 (segment (start 137.16 44.45) (end 136.19432 45.41568) (width 0.1524) (layer "F.Cu") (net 12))
 (segment (start 135.89 66.04) (end 139.7 69.85) (width 0.1524) (layer "F.Cu") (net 14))
 (segment (start 135.89 41.91) (end 135.89 66.04) (width 0.1524) (layer "F.Cu") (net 14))
 (segment (start 133.35 44.196) (end 133.55368 44.39968) (width 0.1524) (layer "F.Cu") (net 16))
 (segment (start 133.35 41.91) (end 133.35 44.196) (width 0.1524) (layer "F.Cu") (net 16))
 (segment (start 134.56968 44.39968) (end 135.58568 45.41568) (width 0.1524) (layer "F.Cu") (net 16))
 (segment (start 135.58568 45.41568) (end 135.58568 68.27568) (width 0.1524) (layer "F.Cu") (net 16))
 (segment (start 135.58568 68.27568) (end 139.7 72.39) (width 0.1524) (layer "F.Cu") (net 16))
 (segment (start 133.55368 44.39968) (end 134.56968 44.39968) (width 0.1524) (layer "F.Cu") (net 16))
 (segment (start 131.064 44.704) (end 134.337746 44.704) (width 0.1524) (layer "F.Cu") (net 18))
 (segment (start 135.28136 70.51136) (end 139.7 74.93) (width 0.1524) (layer "F.Cu") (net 18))
 (segment (start 134.337746 44.704) (end 135.28136 45.647614) (width 0.1524) (layer "F.Cu") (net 18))
 (segment (start 130.81 44.45) (end 131.064 44.704) (width 0.1524) (layer "F.Cu") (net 18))
 (segment (start 135.28136 45.647614) (end 135.28136 70.51136) (width 0.1524) (layer "F.Cu") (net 18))
 (segment (start 130.81 41.91) (end 130.81 44.45) (width 0.1524) (layer "F.Cu") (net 18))
 (segment (start 128.37304 45.06104) (end 134.264412 45.06104) (width 0.1524) (layer "F.Cu") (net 20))
 (segment (start 128.27 41.91) (end 128.27 44.958) (width 0.1524) (layer "F.Cu") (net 20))
 (segment (start 128.27 44.958) (end 128.37304 45.06104) (width 0.1524) (layer "F.Cu") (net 20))
 (segment (start 134.97704 45.773668) (end 134.97704 72.74704) (width 0.1524) (layer "F.Cu") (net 20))
 (segment (start 134.97704 72.74704) (end 139.7 77.47) (width 0.1524) (layer "F.Cu") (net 20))
 (segment (start 134.264412 45.06104) (end 134.97704 45.773668) (width 0.1524) (layer "F.Cu") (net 20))
 (segment (start 125.73 45.212) (end 125.88336 45.36536) (width 0.1524) (layer "F.Cu") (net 22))
 (segment (start 134.138358 45.36536) (end 134.67272 45.899722) (width 0.1524) (layer "F.Cu") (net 22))
 (segment (start 125.88336 45.36536) (end 134.138358 45.36536) (width 0.1524) (layer "F.Cu") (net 22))
 (segment (start 134.67272 45.899722) (end 134.67272 74.98272) (width 0.1524) (layer "F.Cu") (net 22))
 (segment (start 125.73 41.91) (end 125.73 45.212) (width 0.1524) (layer "F.Cu") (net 22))
 (segment (start 134.67272 74.98272) (end 139.7 80.01) (width 0.1524) (layer "F.Cu") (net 22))
 (segment (start 123.19 45.466) (end 123.39368 45.66968) (width 0.1524) (layer "F.Cu") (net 24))
 (segment (start 123.19 41.91) (end 123.19 45.466) (width 0.1524) (layer "F.Cu") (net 24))
 (segment (start 123.39368 45.66968) (end 134.012304 45.66968) (width 0.1524) (layer "F.Cu") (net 24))
 (segment (start 134.3684 46.025776) (end 134.3684 77.2184) (width 0.1524) (layer "F.Cu") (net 24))
 (segment (start 134.012304 45.66968) (end 134.3684 46.025776) (width 0.1524) (layer "F.Cu") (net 24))
 (segment (start 134.3684 77.2184) (end 139.7 82.55) (width 0.1524) (layer "F.Cu") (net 24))
 (segment (start 133.88625 45.974) (end 134.06408 46.15183) (width 0.1524) (layer "F.Cu") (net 26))
 (segment (start 120.65 45.72) (end 120.904 45.974) (width 0.1524) (layer "F.Cu") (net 26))
 (segment (start 120.65 41.91) (end 120.65 45.72) (width 0.1524) (layer "F.Cu") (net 26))
 (segment (start 120.904 45.974) (end 133.88625 45.974) (width 0.1524) (layer "F.Cu") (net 26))
 (segment (start 134.06408 46.15183) (end 134.06408 79.45408) (width 0.1524) (layer "F.Cu") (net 26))
 (segment (start 134.06408 79.45408) (end 139.7 85.09) (width 0.1524) (layer "F.Cu") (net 26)))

